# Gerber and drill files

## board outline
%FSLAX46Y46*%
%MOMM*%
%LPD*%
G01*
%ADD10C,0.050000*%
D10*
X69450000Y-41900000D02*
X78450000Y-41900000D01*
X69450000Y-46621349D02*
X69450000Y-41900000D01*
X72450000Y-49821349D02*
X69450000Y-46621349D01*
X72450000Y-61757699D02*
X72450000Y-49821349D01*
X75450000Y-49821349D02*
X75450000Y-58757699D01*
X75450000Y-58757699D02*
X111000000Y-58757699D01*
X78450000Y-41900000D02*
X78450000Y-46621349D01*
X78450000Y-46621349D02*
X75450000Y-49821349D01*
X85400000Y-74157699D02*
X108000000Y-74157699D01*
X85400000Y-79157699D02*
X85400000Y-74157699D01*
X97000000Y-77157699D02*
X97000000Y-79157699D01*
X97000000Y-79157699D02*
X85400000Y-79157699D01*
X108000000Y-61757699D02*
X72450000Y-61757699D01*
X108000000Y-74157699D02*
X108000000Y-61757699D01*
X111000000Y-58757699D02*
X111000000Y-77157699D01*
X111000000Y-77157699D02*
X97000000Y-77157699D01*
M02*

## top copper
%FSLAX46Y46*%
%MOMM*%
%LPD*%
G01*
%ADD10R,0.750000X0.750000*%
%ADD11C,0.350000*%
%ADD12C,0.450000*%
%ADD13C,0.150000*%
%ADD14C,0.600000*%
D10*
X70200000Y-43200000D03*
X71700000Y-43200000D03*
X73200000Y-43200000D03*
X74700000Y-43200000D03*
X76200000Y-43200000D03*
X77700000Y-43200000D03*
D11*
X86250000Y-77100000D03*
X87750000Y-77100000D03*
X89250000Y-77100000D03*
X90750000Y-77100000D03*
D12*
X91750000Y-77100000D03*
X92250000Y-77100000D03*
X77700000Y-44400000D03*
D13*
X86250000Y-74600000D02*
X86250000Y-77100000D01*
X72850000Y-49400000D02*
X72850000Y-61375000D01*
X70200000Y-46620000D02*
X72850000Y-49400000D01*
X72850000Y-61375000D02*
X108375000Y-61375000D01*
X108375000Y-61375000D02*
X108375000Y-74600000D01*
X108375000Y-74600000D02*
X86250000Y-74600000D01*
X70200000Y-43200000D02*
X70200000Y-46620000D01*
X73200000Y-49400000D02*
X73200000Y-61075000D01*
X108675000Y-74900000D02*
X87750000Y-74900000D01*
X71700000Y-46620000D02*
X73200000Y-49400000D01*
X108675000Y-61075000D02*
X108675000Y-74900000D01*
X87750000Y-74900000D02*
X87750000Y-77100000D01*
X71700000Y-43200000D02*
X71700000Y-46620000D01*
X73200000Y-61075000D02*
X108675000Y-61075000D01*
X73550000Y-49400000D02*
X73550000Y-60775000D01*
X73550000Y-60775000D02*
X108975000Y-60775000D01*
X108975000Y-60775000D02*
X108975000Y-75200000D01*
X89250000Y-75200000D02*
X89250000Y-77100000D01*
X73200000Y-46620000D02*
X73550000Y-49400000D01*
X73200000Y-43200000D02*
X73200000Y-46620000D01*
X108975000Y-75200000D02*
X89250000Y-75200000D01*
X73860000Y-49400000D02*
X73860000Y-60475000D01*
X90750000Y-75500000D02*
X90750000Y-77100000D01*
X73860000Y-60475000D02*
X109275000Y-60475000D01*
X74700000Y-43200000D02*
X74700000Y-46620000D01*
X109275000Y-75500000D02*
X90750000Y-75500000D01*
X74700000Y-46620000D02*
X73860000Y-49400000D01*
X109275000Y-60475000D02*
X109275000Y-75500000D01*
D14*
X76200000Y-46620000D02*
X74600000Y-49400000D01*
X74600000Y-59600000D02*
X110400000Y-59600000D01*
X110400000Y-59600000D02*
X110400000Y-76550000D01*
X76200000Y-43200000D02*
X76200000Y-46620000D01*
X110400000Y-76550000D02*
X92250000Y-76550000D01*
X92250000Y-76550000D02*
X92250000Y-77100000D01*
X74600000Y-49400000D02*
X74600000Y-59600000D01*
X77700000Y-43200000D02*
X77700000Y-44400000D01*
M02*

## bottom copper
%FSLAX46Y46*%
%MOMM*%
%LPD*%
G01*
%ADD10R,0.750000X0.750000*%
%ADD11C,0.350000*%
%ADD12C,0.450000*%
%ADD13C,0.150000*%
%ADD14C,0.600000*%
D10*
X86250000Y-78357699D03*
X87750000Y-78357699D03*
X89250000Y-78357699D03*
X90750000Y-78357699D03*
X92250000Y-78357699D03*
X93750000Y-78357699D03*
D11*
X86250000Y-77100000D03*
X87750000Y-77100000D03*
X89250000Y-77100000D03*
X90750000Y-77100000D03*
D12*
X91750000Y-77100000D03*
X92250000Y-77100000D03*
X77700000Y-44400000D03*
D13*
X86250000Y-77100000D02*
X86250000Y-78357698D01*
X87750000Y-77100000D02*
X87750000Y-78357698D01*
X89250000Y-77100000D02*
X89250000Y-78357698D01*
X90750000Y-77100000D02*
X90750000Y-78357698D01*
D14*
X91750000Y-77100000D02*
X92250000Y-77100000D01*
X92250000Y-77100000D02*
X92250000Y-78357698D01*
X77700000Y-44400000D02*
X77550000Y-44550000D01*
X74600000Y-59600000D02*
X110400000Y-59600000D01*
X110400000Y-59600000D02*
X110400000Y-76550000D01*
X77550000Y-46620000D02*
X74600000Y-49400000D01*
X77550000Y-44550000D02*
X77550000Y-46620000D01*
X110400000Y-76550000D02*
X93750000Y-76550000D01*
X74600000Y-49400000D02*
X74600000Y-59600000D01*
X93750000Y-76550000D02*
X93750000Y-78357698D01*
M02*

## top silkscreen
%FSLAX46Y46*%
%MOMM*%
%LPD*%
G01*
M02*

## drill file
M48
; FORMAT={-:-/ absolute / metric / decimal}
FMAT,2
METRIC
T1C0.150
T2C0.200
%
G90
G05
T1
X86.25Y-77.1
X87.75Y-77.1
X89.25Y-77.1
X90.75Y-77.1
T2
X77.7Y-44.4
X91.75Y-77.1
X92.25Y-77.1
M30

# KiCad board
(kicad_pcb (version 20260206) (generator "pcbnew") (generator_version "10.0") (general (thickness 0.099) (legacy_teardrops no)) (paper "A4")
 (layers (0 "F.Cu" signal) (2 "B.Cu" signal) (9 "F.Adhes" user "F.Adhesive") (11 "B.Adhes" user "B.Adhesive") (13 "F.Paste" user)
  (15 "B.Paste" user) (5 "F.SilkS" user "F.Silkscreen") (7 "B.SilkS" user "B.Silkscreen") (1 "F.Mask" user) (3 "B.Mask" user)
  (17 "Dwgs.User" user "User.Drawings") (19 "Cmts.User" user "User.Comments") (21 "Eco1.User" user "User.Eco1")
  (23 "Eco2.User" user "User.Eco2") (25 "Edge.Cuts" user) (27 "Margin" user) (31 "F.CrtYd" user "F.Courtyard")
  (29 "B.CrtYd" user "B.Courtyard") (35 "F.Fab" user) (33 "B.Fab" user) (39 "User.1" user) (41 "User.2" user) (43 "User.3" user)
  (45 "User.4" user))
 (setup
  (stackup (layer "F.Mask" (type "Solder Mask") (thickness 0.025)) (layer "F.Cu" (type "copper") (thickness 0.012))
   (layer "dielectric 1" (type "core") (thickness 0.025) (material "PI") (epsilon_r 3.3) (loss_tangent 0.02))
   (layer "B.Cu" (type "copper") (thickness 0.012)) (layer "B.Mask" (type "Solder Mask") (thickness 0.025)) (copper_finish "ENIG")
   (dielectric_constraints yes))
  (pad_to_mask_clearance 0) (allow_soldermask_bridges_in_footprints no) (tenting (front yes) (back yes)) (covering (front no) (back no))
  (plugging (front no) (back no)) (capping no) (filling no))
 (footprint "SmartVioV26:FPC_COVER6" (layer "F.Cu") (at 0 0)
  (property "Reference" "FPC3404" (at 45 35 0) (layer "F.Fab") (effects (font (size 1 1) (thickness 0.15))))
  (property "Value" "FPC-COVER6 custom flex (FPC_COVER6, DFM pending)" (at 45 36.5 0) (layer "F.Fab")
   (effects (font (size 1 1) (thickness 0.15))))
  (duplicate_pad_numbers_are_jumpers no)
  (pad "S1" smd rect (at 70.2 43.2) (size 0.75 0.75) (layers "F.Cu" "F.Mask") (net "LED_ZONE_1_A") (solder_mask_margin 0.1))
  (pad "S2" smd rect (at 71.7 43.2) (size 0.75 0.75) (layers "F.Cu" "F.Mask") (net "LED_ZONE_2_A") (solder_mask_margin 0.1))
  (pad "S3" smd rect (at 73.2 43.2) (size 0.75 0.75) (layers "F.Cu" "F.Mask") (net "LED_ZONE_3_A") (solder_mask_margin 0.1))
  (pad "S4" smd rect (at 74.7 43.2) (size 0.75 0.75) (layers "F.Cu" "F.Mask") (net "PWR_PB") (solder_mask_margin 0.1))
  (pad "S5" smd rect (at 76.2 43.2) (size 0.75 0.75) (layers "F.Cu" "F.Mask") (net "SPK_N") (solder_mask_margin 0.1))
  (pad "S6" smd rect (at 77.7 43.2) (size 0.75 0.75) (layers "F.Cu" "F.Mask") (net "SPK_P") (solder_mask_margin 0.1))
  (pad "T1" smd rect (at 86.25 78.357699) (size 0.75 0.75) (layers "B.Cu" "B.Mask") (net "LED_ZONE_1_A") (solder_mask_margin 0.1))
  (pad "T2" smd rect (at 87.75 78.357699) (size 0.75 0.75) (layers "B.Cu" "B.Mask") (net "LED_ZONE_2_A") (solder_mask_margin 0.1))
  (pad "T3" smd rect (at 89.25 78.357699) (size 0.75 0.75) (layers "B.Cu" "B.Mask") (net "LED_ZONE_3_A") (solder_mask_margin 0.1))
  (pad "T4" smd rect (at 90.75 78.357699) (size 0.75 0.75) (layers "B.Cu" "B.Mask") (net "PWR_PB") (solder_mask_margin 0.1))
  (pad "T5" smd rect (at 92.25 78.357699) (size 0.75 0.75) (layers "B.Cu" "B.Mask") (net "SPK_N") (solder_mask_margin 0.1))
  (pad "T6" smd rect (at 93.75 78.357699) (size 0.75 0.75) (layers "B.Cu" "B.Mask") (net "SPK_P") (solder_mask_margin 0.1)))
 (gr_line (start 69.45 41.9) (end 78.45 41.9) (stroke (width 0.05) (type default)) (layer "Edge.Cuts"))
 (gr_line (start 69.45 46.621349) (end 69.45 41.9) (stroke (width 0.05) (type default)) (layer "Edge.Cuts"))
 (gr_line (start 72.45 49.821349) (end 69.45 46.621349) (stroke (width 0.05) (type default)) (layer "Edge.Cuts"))
 (gr_line (start 72.45 61.757699) (end 72.45 49.821349) (stroke (width 0.05) (type default)) (layer "Edge.Cuts"))
 (gr_line (start 75.45 49.821349) (end 75.45 58.757699) (stroke (width 0.05) (type default)) (layer "Edge.Cuts"))
 (gr_line (start 75.45 58.757699) (end 111 58.757699) (stroke (width 0.05) (type default)) (layer "Edge.Cuts"))
 (gr_line (start 78.45 41.9) (end 78.45 46.621349) (stroke (width 0.05) (type default)) (layer "Edge.Cuts"))
 (gr_line (start 78.45 46.621349) (end 75.45 49.821349) (stroke (width 0.05) (type default)) (layer "Edge.Cuts"))
 (gr_line (start 85.4 74.157699) (end 108 74.157699) (stroke (width 0.05) (type default)) (layer "Edge.Cuts"))
 (gr_line (start 85.4 79.157699) (end 85.4 74.157699) (stroke (width 0.05) (type default)) (layer "Edge.Cuts"))
 (gr_line (start 97 77.157699) (end 97 79.157699) (stroke (width 0.05) (type default)) (layer "Edge.Cuts"))
 (gr_line (start 97 79.157699) (end 85.4 79.157699) (stroke (width 0.05) (type default)) (layer "Edge.Cuts"))
 (gr_line (start 108 61.757699) (end 72.45 61.757699) (stroke (width 0.05) (type default)) (layer "Edge.Cuts"))
 (gr_line (start 108 74.157699) (end 108 61.757699) (stroke (width 0.05) (type default)) (layer "Edge.Cuts"))
 (gr_line (start 111 58.757699) (end 111 77.157699) (stroke (width 0.05) (type default)) (layer "Edge.Cuts"))
 (gr_line (start 111 77.157699) (end 97 77.157699) (stroke (width 0.05) (type default)) (layer "Edge.Cuts"))
 (segment (start 86.25 74.6) (end 86.25 77.1) (width 0.15) (layer "F.Cu") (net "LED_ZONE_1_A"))
 (segment (start 72.85 49.4) (end 72.85 61.375) (width 0.15) (layer "F.Cu") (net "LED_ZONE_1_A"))
 (segment (start 70.2 46.62) (end 72.85 49.4) (width 0.15) (layer "F.Cu") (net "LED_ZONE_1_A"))
 (segment (start 72.85 61.375) (end 108.375 61.375) (width 0.15) (layer "F.Cu") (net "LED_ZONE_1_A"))
 (segment (start 108.375 61.375) (end 108.375 74.6) (width 0.15) (layer "F.Cu") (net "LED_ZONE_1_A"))
 (segment (start 108.375 74.6) (end 86.25 74.6) (width 0.15) (layer "F.Cu") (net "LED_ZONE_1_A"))
 (segment (start 70.2 43.2) (end 70.2 46.62) (width 0.15) (layer "F.Cu") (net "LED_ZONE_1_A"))
 (via (at 86.25 77.1) (size 0.35) (drill 0.15) (layers "F.Cu" "B.Cu") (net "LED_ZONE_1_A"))
 (segment (start 86.25 77.1) (end 86.25 78.357698) (width 0.15) (layer "B.Cu") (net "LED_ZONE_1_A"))
 (segment (start 73.2 49.4) (end 73.2 61.075) (width 0.15) (layer "F.Cu") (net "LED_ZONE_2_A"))
 (segment (start 108.675 74.9) (end 87.75 74.9) (width 0.15) (layer "F.Cu") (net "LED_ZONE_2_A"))
 (segment (start 71.7 46.62) (end 73.2 49.4) (width 0.15) (layer "F.Cu") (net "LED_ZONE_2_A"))
 (segment (start 108.675 61.075) (end 108.675 74.9) (width 0.15) (layer "F.Cu") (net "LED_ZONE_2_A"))
 (segment (start 87.75 74.9) (end 87.75 77.1) (width 0.15) (layer "F.Cu") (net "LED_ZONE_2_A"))
 (segment (start 71.7 43.2) (end 71.7 46.62) (width 0.15) (layer "F.Cu") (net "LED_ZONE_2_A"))
 (segment (start 73.2 61.075) (end 108.675 61.075) (width 0.15) (layer "F.Cu") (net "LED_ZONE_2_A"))
 (via (at 87.75 77.1) (size 0.35) (drill 0.15) (layers "F.Cu" "B.Cu") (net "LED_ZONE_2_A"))
 (segment (start 87.75 77.1) (end 87.75 78.357698) (width 0.15) (layer "B.Cu") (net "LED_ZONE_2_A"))
 (segment (start 73.55 49.4) (end 73.55 60.775) (width 0.15) (layer "F.Cu") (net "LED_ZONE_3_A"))
 (segment (start 73.55 60.775) (end 108.975 60.775) (width 0.15) (layer "F.Cu") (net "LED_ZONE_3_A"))
 (segment (start 108.975 60.775) (end 108.975 75.2) (width 0.15) (layer "F.Cu") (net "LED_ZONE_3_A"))
 (segment (start 89.25 75.2) (end 89.25 77.1) (width 0.15) (layer "F.Cu") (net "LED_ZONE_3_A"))
 (segment (start 73.2 46.62) (end 73.55 49.4) (width 0.15) (layer "F.Cu") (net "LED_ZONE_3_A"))
 (segment (start 73.2 43.2) (end 73.2 46.62) (width 0.15) (layer "F.Cu") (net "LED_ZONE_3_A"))
 (segment (start 108.975 75.2) (end 89.25 75.2) (width 0.15) (layer "F.Cu") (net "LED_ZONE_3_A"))
 (via (at 89.25 77.1) (size 0.35) (drill 0.15) (layers "F.Cu" "B.Cu") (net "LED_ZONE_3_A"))
 (segment (start 89.25 77.1) (end 89.25 78.357698) (width 0.15) (layer "B.Cu") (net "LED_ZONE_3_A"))
 (segment (start 73.86 49.4) (end 73.86 60.475) (width 0.15) (layer "F.Cu") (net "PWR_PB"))
 (segment (start 90.75 75.5) (end 90.75 77.1) (width 0.15) (layer "F.Cu") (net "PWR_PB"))
 (segment (start 73.86 60.475) (end 109.275 60.475) (width 0.15) (layer "F.Cu") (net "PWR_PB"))
 (segment (start 74.7 43.2) (end 74.7 46.62) (width 0.15) (layer "F.Cu") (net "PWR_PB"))
 (segment (start 109.275 75.5) (end 90.75 75.5) (width 0.15) (layer "F.Cu") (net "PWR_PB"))
 (segment (start 74.7 46.62) (end 73.86 49.4) (width 0.15) (layer "F.Cu") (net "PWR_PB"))
 (segment (start 109.275 60.475) (end 109.275 75.5) (width 0.15) (layer "F.Cu") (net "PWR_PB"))
 (via (at 90.75 77.1) (size 0.35) (drill 0.15) (layers "F.Cu" "B.Cu") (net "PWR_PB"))
 (segment (start 90.75 77.1) (end 90.75 78.357698) (width 0.15) (layer "B.Cu") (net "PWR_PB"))
 (segment (start 76.2 46.62) (end 74.6 49.4) (width 0.6) (layer "F.Cu") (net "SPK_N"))
 (segment (start 74.6 59.6) (end 110.4 59.6) (width 0.6) (layer "F.Cu") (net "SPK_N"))
 (segment (start 110.4 59.6) (end 110.4 76.55) (width 0.6) (layer "F.Cu") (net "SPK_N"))
 (segment (start 76.2 43.2) (end 76.2 46.62) (width 0.6) (layer "F.Cu") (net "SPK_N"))
 (segment (start 110.4 76.55) (end 92.25 76.55) (width 0.6) (layer "F.Cu") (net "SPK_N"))
 (segment (start 92.25 76.55) (end 92.25 77.1) (width 0.6) (layer "F.Cu") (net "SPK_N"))
 (segment (start 74.6 49.4) (end 74.6 59.6) (width 0.6) (layer "F.Cu") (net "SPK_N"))
 (via (at 91.75 77.1) (size 0.45) (drill 0.2) (layers "F.Cu" "B.Cu") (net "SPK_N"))
 (via (at 92.25 77.1) (size 0.45) (drill 0.2) (layers "F.Cu" "B.Cu") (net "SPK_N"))
 (segment (start 91.75 77.1) (end 92.25 77.1) (width 0.6) (layer "B.Cu") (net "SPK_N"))
 (segment (start 92.25 77.1) (end 92.25 78.357698) (width 0.6) (layer "B.Cu") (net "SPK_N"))
 (segment (start 77.7 43.2) (end 77.7 44.4) (width 0.6) (layer "F.Cu") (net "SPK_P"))
 (via (at 77.7 44.4) (size 0.45) (drill 0.2) (layers "F.Cu" "B.Cu") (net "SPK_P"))
 (segment (start 77.7 44.4) (end 77.55 44.55) (width 0.6) (layer "B.Cu") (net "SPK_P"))
 (segment (start 74.6 59.6) (end 110.4 59.6) (width 0.6) (layer "B.Cu") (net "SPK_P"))
 (segment (start 110.4 59.6) (end 110.4 76.55) (width 0.6) (layer "B.Cu") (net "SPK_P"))
 (segment (start 77.55 46.62) (end 74.6 49.4) (width 0.6) (layer "B.Cu") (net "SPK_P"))
 (segment (start 77.55 44.55) (end 77.55 46.62) (width 0.6) (layer "B.Cu") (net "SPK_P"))
 (segment (start 110.4 76.55) (end 93.75 76.55) (width 0.6) (layer "B.Cu") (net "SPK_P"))
 (segment (start 74.6 49.4) (end 74.6 59.6) (width 0.6) (layer "B.Cu") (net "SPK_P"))
 (segment (start 93.75 76.55) (end 93.75 78.357698) (width 0.6) (layer "B.Cu") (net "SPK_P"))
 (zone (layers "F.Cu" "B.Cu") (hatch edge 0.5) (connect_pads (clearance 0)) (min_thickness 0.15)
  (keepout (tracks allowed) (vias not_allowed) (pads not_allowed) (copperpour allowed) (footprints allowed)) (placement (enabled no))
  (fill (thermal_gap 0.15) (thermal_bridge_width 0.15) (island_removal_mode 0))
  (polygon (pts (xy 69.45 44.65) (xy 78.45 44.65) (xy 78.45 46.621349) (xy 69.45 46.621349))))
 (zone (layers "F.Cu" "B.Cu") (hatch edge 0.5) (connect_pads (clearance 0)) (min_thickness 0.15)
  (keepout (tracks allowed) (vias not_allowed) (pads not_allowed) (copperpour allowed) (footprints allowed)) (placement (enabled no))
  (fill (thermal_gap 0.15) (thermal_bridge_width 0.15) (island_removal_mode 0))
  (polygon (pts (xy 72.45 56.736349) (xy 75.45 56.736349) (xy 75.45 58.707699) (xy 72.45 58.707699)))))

